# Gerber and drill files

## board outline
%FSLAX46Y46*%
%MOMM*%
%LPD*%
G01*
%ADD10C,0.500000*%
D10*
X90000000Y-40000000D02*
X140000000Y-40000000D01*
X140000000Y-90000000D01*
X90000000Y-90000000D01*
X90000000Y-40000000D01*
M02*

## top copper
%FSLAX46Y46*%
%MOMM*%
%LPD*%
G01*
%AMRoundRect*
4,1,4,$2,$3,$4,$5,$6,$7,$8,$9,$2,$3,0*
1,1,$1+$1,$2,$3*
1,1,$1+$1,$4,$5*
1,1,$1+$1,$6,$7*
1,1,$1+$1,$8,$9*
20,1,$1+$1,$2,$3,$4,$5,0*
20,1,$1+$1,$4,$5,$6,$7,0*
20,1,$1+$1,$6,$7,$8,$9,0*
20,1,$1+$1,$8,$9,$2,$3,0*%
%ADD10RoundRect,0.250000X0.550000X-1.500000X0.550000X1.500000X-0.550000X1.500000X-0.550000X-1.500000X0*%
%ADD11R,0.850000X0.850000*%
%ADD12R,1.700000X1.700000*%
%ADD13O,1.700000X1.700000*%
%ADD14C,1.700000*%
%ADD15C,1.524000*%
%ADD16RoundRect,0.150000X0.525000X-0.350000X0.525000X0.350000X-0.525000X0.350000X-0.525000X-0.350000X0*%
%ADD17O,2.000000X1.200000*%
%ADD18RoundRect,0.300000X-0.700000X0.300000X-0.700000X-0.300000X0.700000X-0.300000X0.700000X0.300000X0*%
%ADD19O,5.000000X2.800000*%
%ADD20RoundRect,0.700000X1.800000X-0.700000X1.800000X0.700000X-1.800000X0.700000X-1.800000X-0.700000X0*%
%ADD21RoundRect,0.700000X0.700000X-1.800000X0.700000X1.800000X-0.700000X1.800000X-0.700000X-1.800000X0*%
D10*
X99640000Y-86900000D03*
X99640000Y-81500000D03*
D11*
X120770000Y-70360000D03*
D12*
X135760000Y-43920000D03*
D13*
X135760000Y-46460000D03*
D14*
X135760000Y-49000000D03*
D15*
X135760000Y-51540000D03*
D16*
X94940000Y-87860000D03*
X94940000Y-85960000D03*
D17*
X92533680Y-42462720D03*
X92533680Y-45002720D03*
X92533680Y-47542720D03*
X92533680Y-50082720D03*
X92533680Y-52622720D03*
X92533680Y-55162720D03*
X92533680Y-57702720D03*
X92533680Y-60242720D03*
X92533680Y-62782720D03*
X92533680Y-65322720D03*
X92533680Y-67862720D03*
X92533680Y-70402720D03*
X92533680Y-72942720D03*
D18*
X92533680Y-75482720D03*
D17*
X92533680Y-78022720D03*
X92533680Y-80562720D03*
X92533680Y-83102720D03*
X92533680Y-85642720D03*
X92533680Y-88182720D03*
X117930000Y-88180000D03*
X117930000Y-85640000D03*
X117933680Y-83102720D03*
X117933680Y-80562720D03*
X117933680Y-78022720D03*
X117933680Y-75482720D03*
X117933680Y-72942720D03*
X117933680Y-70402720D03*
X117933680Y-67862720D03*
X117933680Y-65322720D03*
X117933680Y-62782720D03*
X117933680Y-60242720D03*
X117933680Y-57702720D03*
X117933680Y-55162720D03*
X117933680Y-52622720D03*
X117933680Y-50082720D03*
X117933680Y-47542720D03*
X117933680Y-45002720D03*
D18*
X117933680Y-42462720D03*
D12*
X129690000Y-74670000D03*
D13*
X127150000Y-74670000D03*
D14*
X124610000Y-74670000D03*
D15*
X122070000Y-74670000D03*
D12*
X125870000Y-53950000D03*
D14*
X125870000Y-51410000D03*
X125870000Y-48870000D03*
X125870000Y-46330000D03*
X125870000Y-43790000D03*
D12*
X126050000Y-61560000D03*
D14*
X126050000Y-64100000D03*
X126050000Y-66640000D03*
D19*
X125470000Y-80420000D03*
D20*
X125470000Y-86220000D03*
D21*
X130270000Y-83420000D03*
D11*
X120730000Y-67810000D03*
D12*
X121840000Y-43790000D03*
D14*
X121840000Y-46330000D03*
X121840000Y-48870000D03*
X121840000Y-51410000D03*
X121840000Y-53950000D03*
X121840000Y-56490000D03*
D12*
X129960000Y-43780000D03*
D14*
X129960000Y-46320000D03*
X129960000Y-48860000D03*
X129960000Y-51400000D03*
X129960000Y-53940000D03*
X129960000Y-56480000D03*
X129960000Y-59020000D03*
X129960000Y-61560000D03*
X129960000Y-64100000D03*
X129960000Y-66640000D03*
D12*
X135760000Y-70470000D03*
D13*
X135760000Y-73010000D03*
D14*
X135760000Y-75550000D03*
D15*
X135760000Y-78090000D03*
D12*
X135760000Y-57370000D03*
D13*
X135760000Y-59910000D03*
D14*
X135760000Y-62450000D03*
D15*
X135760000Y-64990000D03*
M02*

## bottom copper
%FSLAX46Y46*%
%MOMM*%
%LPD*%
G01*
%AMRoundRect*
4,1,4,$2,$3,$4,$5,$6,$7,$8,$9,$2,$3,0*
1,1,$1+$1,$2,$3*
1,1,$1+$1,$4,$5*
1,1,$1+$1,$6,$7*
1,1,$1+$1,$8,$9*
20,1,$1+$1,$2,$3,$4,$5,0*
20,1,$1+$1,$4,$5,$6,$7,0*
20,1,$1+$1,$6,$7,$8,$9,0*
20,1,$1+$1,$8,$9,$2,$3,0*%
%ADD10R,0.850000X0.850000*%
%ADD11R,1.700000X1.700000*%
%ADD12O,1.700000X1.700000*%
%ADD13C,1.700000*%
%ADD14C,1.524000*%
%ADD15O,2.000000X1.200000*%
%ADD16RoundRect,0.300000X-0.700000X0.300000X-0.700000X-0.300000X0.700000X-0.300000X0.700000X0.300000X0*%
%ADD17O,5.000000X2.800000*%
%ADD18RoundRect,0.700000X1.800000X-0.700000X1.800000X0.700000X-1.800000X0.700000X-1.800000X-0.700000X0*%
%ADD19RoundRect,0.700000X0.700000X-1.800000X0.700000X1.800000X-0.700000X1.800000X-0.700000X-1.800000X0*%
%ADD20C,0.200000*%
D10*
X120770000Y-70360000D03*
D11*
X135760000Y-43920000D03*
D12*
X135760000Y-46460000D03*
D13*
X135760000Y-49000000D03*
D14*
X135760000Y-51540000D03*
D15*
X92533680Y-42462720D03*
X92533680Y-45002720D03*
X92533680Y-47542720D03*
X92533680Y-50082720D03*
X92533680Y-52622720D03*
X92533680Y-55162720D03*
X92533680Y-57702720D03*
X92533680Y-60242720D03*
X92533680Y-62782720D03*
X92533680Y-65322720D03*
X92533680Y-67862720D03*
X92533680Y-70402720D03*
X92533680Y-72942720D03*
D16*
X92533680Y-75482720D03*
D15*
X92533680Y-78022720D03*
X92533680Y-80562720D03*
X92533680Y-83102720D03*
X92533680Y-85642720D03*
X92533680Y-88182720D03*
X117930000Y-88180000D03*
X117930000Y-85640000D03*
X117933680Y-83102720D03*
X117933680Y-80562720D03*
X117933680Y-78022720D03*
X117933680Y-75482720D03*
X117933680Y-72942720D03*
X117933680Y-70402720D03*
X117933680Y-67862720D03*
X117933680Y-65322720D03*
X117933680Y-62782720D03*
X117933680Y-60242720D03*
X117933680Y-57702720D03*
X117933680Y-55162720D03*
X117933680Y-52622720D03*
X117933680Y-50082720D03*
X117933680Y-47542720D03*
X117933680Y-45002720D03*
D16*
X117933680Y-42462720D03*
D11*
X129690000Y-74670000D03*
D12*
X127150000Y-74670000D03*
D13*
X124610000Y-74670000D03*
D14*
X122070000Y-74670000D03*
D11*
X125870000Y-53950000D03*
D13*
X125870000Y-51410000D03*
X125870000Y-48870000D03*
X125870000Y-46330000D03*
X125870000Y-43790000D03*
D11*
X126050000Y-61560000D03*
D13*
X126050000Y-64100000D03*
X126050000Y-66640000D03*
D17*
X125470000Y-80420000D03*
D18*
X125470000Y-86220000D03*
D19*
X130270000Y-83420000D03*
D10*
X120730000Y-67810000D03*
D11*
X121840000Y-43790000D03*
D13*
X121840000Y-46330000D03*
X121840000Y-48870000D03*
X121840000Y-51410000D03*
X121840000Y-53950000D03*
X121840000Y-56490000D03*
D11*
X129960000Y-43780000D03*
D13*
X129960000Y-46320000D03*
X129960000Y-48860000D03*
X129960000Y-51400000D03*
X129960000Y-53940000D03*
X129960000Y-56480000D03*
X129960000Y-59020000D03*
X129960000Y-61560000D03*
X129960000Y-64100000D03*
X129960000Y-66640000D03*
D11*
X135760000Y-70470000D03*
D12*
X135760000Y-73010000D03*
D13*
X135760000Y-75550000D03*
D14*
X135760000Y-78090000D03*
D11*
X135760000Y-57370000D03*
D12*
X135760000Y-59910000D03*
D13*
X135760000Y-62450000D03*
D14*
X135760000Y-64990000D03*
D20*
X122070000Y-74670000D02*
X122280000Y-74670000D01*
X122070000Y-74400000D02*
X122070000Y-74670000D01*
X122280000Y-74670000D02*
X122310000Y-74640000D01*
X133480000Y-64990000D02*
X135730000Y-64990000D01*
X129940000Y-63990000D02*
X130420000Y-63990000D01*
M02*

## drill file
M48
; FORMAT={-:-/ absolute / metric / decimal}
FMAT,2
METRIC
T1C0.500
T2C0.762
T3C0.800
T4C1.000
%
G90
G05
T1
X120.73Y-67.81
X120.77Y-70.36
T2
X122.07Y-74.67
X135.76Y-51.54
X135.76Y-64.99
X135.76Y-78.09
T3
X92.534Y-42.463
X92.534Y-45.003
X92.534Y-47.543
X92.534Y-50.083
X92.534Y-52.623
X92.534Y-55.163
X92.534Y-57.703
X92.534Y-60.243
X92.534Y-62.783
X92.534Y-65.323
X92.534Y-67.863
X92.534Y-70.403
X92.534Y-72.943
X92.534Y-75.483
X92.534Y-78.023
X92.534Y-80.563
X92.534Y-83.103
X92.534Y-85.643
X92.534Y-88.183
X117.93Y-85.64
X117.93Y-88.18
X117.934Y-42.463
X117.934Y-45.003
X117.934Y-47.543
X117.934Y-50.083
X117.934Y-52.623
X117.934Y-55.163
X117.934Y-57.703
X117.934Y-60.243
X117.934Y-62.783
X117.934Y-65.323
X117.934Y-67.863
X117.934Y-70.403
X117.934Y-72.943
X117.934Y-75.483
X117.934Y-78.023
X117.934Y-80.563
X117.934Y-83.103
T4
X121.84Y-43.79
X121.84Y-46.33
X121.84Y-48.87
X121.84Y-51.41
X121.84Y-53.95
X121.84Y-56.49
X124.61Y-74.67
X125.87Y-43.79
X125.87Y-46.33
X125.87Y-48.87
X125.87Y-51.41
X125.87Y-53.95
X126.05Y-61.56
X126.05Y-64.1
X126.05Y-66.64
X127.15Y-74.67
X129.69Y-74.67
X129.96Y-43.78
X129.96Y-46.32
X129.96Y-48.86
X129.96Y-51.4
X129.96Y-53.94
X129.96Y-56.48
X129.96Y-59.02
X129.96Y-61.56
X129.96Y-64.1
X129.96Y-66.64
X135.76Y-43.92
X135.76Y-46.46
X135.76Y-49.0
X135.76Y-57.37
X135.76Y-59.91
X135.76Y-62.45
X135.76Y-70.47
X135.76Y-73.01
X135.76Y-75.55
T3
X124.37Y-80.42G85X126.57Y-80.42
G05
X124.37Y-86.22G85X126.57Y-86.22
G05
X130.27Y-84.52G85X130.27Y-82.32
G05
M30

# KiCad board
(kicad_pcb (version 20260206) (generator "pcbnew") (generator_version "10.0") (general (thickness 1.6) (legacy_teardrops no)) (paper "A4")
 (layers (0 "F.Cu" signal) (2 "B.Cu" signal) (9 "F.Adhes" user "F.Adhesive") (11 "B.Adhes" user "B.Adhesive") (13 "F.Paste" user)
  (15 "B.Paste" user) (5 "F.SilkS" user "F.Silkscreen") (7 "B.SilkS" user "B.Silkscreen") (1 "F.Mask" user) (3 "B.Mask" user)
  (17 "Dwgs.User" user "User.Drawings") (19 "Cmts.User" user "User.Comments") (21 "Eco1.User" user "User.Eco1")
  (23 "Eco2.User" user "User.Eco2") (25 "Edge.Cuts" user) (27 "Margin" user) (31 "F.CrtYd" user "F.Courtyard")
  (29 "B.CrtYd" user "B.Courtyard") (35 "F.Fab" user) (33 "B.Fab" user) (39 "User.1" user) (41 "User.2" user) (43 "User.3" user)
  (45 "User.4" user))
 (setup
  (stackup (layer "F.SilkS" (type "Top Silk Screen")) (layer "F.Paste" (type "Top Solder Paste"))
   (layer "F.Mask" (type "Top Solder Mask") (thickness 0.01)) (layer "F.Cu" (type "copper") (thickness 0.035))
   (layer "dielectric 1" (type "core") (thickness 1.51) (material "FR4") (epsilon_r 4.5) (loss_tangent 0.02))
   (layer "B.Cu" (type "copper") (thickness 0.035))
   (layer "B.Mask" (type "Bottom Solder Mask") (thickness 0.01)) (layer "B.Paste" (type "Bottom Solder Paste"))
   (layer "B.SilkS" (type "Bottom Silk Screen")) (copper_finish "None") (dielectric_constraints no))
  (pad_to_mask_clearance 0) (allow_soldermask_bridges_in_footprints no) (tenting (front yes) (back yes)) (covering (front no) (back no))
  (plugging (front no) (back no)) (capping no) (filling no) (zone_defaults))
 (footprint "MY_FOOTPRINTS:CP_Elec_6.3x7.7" (layer "F.Cu") (at 99.64 84.2 90)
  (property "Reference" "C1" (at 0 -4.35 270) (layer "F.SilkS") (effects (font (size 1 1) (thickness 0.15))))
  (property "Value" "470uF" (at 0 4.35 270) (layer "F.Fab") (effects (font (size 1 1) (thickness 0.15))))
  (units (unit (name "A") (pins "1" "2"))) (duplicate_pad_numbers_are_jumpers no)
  (pad "1" smd roundrect (at -2.7 0 90) (size 3.5 1.6) (layers "F.Cu" "F.Mask" "F.Paste") (roundrect_rratio 0.15625) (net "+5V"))
  (pad "2" smd roundrect (at 2.7 0 90) (size 3.5 1.6) (layers "F.Cu" "F.Mask" "F.Paste") (roundrect_rratio 0.15625) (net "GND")))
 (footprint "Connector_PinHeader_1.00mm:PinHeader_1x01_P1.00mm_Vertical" (layer "F.Cu") (at 120.77 70.36)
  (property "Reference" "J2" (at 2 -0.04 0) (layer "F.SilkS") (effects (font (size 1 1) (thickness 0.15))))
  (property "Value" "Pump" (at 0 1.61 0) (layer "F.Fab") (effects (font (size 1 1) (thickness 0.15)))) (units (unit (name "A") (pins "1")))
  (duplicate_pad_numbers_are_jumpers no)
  (pad "1" thru_hole rect (at 0 0) (size 0.85 0.85) (drill 0.5) (layers "*.Cu" "*.Mask") (remove_unused_layers no) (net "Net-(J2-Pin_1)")))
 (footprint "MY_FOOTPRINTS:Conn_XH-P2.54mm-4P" (layer "F.Cu") (at 135.76 47.73)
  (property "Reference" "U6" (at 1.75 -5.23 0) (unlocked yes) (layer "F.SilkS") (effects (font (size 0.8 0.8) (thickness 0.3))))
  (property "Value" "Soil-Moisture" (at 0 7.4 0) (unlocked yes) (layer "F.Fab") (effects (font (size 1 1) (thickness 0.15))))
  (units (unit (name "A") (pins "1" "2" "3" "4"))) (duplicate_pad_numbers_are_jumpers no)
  (pad "1" thru_hole rect (at 0 -3.81) (size 1.7 1.7) (drill 1) (layers "*.Cu" "*.Mask") (remove_unused_layers no) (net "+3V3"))
  (pad "2" thru_hole oval (at 0 -1.27) (size 1.7 1.7) (drill 1) (layers "*.Cu" "*.Mask") (remove_unused_layers no) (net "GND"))
  (pad "3" thru_hole circle (at 0 1.27) (size 1.7 1.7) (drill 1) (layers "*.Cu" "*.Mask") (remove_unused_layers no)
   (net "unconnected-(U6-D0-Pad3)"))
  (pad "4" thru_hole circle (at 0 3.81) (size 1.524 1.524) (drill 0.762) (layers "*.Cu" "*.Mask") (remove_unused_layers no)
   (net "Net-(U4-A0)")))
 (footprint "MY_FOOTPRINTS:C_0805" (layer "F.Cu") (at 94.94 86.91 90)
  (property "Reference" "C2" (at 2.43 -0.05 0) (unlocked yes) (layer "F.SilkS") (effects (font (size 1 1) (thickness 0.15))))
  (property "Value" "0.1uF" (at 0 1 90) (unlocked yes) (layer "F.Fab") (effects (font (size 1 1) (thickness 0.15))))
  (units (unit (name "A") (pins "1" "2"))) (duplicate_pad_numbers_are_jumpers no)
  (pad "1" smd roundrect (at -0.95 0 90) (size 1 1.35) (layers "F.Cu" "F.Mask" "F.Paste") (roundrect_rratio 0.15) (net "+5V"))
  (pad "2" smd roundrect (at 0.95 0 90) (size 1 1.35) (layers "F.Cu" "F.Mask" "F.Paste") (roundrect_rratio 0.15) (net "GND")))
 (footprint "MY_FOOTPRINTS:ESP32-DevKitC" (layer "F.Cu") (at 92.53 42.46)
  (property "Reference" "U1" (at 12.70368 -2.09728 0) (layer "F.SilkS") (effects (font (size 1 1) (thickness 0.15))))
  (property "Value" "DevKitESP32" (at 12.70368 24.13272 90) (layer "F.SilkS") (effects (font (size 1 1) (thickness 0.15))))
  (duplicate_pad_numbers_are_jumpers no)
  (pad "1" thru_hole oval (at 0.00368 0.00272 270) (size 1.2 2) (drill 0.8) (layers "*.Cu" "*.Mask") (remove_unused_layers no) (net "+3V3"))
  (pad "2" thru_hole oval (at 0.00368 2.54272 270) (size 1.2 2) (drill 0.8) (layers "*.Cu" "*.Mask") (remove_unused_layers no)
   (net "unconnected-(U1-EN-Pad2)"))
  (pad "3" thru_hole oval (at 0.00368 5.08272 270) (size 1.2 2) (drill 0.8) (layers "*.Cu" "*.Mask") (remove_unused_layers no)
   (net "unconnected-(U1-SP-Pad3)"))
  (pad "4" thru_hole oval (at 0.00368 7.62272 270) (size 1.2 2) (drill 0.8) (layers "*.Cu" "*.Mask") (remove_unused_layers no)
   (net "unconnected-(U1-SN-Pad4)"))
  (pad "5" thru_hole oval (at 0.00368 10.16272 270) (size 1.2 2) (drill 0.8) (layers "*.Cu" "*.Mask") (remove_unused_layers no)
   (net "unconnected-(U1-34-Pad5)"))
  (pad "6" thru_hole oval (at 0.00368 12.70272 270) (size 1.2 2) (drill 0.8) (layers "*.Cu" "*.Mask") (remove_unused_layers no)
   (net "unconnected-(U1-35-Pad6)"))
  (pad "7" thru_hole oval (at 0.00368 15.24272 270) (size 1.2 2) (drill 0.8) (layers "*.Cu" "*.Mask") (remove_unused_layers no)
   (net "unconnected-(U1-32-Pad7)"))
  (pad "8" thru_hole oval (at 0.00368 17.78272 270) (size 1.2 2) (drill 0.8) (layers "*.Cu" "*.Mask") (remove_unused_layers no)
   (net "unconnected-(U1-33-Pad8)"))
  (pad "9" thru_hole oval (at 0.00368 20.32272 270) (size 1.2 2) (drill 0.8) (layers "*.Cu" "*.Mask") (remove_unused_layers no)
   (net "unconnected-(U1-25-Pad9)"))
  (pad "10" thru_hole oval (at 0.00368 22.86272 270) (size 1.2 2) (drill 0.8) (layers "*.Cu" "*.Mask") (remove_unused_layers no)
   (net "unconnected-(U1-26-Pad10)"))
  (pad "11" thru_hole oval (at 0.00368 25.40272 270) (size 1.2 2) (drill 0.8) (layers "*.Cu" "*.Mask") (remove_unused_layers no)
   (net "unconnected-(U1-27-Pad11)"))
  (pad "12" thru_hole oval (at 0.00368 27.94272 270) (size 1.2 2) (drill 0.8) (layers "*.Cu" "*.Mask") (remove_unused_layers no)
   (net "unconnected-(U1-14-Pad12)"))
  (pad "13" thru_hole oval (at 0.00368 30.48272 270) (size 1.2 2) (drill 0.8) (layers "*.Cu" "*.Mask") (remove_unused_layers no)
   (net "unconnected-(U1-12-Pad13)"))
  (pad "14" thru_hole roundrect (at 0.00368 33.02272 270) (size 1.2 2) (drill 0.8) (layers "*.Cu" "*.Mask") (remove_unused_layers no)
   (roundrect_rratio 0.25) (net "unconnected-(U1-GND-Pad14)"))
  (pad "15" thru_hole oval (at 0.00368 35.56272 270) (size 1.2 2) (drill 0.8) (layers "*.Cu" "*.Mask") (remove_unused_layers no)
   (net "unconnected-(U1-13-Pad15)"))
  (pad "16" thru_hole oval (at 0.00368 38.10272 270) (size 1.2 2) (drill 0.8) (layers "*.Cu" "*.Mask") (remove_unused_layers no)
   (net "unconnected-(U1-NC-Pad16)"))
  (pad "17" thru_hole oval (at 0.00368 40.64272 270) (size 1.2 2) (drill 0.8) (layers "*.Cu" "*.Mask") (remove_unused_layers no)
   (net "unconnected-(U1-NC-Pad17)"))
  (pad "18" thru_hole oval (at 0.00368 43.18272 270) (size 1.2 2) (drill 0.8) (layers "*.Cu" "*.Mask") (remove_unused_layers no) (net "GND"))
  (pad "19" thru_hole oval (at 0.00368 45.72272 270) (size 1.2 2) (drill 0.8) (layers "*.Cu" "*.Mask") (remove_unused_layers no) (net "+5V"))
  (pad "20" thru_hole oval (at 25.4 45.72 270) (size 1.2 2) (drill 0.8) (layers "*.Cu" "*.Mask") (remove_unused_layers no)
   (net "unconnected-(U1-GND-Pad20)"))
  (pad "21" thru_hole oval (at 25.4 43.18 270) (size 1.2 2) (drill 0.8) (layers "*.Cu" "*.Mask") (remove_unused_layers no)
   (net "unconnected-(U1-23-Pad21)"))
  (pad "22" thru_hole oval (at 25.40368 40.64272 270) (size 1.2 2) (drill 0.8) (layers "*.Cu" "*.Mask") (remove_unused_layers no)
   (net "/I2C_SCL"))
  (pad "23" thru_hole oval (at 25.40368 38.10272 270) (size 1.2 2) (drill 0.8) (layers "*.Cu" "*.Mask") (remove_unused_layers no)
   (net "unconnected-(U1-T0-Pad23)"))
  (pad "24" thru_hole oval (at 25.40368 35.56272 270) (size 1.2 2) (drill 0.8) (layers "*.Cu" "*.Mask") (remove_unused_layers no)
   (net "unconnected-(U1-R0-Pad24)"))
  (pad "25" thru_hole oval (at 25.40368 33.02272 270) (size 1.2 2) (drill 0.8) (layers "*.Cu" "*.Mask") (remove_unused_layers no)
   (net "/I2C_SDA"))
  (pad "26" thru_hole oval (at 25.40368 30.48272 270) (size 1.2 2) (drill 0.8) (layers "*.Cu" "*.Mask") (remove_unused_layers no)
   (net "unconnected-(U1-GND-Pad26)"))
  (pad "27" thru_hole oval (at 25.40368 27.94272 270) (size 1.2 2) (drill 0.8) (layers "*.Cu" "*.Mask") (remove_unused_layers no)
   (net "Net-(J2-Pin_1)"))
  (pad "28" thru_hole oval (at 25.40368 25.40272 270) (size 1.2 2) (drill 0.8) (layers "*.Cu" "*.Mask") (remove_unused_layers no)
   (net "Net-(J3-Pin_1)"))
  (pad "29" thru_hole oval (at 25.40368 22.86272 270) (size 1.2 2) (drill 0.8) (layers "*.Cu" "*.Mask") (remove_unused_layers no)
   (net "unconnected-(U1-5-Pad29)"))
  (pad "30" thru_hole oval (at 25.40368 20.32272 270) (size 1.2 2) (drill 0.8) (layers "*.Cu" "*.Mask") (remove_unused_layers no)
   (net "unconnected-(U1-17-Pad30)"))
  (pad "31" thru_hole oval (at 25.40368 17.78272 270) (size 1.2 2) (drill 0.8) (layers "*.Cu" "*.Mask") (remove_unused_layers no)
   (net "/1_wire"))
  (pad "32" thru_hole oval (at 25.40368 15.24272 270) (size 1.2 2) (drill 0.8) (layers "*.Cu" "*.Mask") (remove_unused_layers no)
   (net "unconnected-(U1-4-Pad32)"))
  (pad "33" thru_hole oval (at 25.40368 12.70272 270) (size 1.2 2) (drill 0.8) (layers "*.Cu" "*.Mask") (remove_unused_layers no)
   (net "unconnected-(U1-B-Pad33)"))
  (pad "34" thru_hole oval (at 25.40368 10.16272 270) (size 1.2 2) (drill 0.8) (layers "*.Cu" "*.Mask") (remove_unused_layers no)
   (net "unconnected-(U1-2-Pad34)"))
  (pad "35" thru_hole oval (at 25.40368 7.62272 270) (size 1.2 2) (drill 0.8) (layers "*.Cu" "*.Mask") (remove_unused_layers no)
   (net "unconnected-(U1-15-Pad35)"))
  (pad "36" thru_hole oval (at 25.40368 5.08272 270) (size 1.2 2) (drill 0.8) (layers "*.Cu" "*.Mask") (remove_unused_layers no)
   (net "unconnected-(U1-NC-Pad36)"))
  (pad "37" thru_hole oval (at 25.40368 2.54272 270) (size 1.2 2) (drill 0.8) (layers "*.Cu" "*.Mask") (remove_unused_layers no)
   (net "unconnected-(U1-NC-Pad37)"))
  (pad "38" thru_hole roundrect (at 25.40368 0.00272 270) (size 1.2 2) (drill 0.8) (layers "*.Cu" "*.Mask") (remove_unused_layers no)
   (roundrect_rratio 0.25) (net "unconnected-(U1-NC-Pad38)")))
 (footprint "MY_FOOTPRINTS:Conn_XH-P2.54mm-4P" (layer "F.Cu") (at 125.88 74.67 -90)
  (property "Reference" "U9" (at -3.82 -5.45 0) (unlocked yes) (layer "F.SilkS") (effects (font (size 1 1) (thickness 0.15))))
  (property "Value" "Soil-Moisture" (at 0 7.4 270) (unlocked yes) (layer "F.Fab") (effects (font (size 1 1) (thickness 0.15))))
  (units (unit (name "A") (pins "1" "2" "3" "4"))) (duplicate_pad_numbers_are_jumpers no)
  (pad "1" thru_hole rect (at 0 -3.81 270) (size 1.7 1.7) (drill 1) (layers "*.Cu" "*.Mask") (remove_unused_layers no) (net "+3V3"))
  (pad "2" thru_hole oval (at 0 -1.27 270) (size 1.7 1.7) (drill 1) (layers "*.Cu" "*.Mask") (remove_unused_layers no) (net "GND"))
  (pad "3" thru_hole circle (at 0 1.27 270) (size 1.7 1.7) (drill 1) (layers "*.Cu" "*.Mask") (remove_unused_layers no)
   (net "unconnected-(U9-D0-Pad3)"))
  (pad "4" thru_hole circle (at 0 3.81 270) (size 1.524 1.524) (drill 0.762) (layers "*.Cu" "*.Mask") (remove_unused_layers no)
   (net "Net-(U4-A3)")))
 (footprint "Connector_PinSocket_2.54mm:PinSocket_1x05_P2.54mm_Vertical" (layer "F.Cu") (at 125.87 53.95 180)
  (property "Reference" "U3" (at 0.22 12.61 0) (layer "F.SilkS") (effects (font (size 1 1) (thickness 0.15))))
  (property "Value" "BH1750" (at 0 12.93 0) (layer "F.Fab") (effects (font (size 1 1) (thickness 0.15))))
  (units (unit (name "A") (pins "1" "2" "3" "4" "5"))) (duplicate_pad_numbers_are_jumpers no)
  (pad "1" thru_hole rect (at 0 0 180) (size 1.7 1.7) (drill 1) (layers "*.Cu" "*.Mask") (remove_unused_layers no) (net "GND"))
  (pad "2" thru_hole circle (at 0 2.54 180) (size 1.7 1.7) (drill 1) (layers "*.Cu" "*.Mask") (remove_unused_layers no)
   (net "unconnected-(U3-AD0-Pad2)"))
  (pad "3" thru_hole circle (at 0 5.08 180) (size 1.7 1.7) (drill 1) (layers "*.Cu" "*.Mask") (remove_unused_layers no) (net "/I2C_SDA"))
  (pad "4" thru_hole circle (at 0 7.62 180) (size 1.7 1.7) (drill 1) (layers "*.Cu" "*.Mask") (remove_unused_layers no) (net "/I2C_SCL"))
  (pad "5" thru_hole circle (at 0 10.16 180) (size 1.7 1.7) (drill 1) (layers "*.Cu" "*.Mask") (remove_unused_layers no) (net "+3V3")))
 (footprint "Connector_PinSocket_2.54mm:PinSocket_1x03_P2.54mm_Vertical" (layer "F.Cu") (at 126.05 61.56)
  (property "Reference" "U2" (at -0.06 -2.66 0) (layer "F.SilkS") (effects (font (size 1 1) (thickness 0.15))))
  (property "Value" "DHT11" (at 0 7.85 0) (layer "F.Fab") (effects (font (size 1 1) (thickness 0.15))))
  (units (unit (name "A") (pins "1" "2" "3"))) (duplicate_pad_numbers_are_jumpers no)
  (pad "1" thru_hole rect (at 0 0) (size 1.7 1.7) (drill 1) (layers "*.Cu" "*.Mask") (remove_unused_layers no) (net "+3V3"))
  (pad "2" thru_hole circle (at 0 2.54) (size 1.7 1.7) (drill 1) (layers "*.Cu" "*.Mask") (remove_unused_layers no) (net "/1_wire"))
  (pad "3" thru_hole circle (at 0 5.08) (size 1.7 1.7) (drill 1) (layers "*.Cu" "*.Mask") (remove_unused_layers no) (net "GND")))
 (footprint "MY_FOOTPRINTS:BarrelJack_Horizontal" (layer "F.Cu") (at 125.47 80.42 90)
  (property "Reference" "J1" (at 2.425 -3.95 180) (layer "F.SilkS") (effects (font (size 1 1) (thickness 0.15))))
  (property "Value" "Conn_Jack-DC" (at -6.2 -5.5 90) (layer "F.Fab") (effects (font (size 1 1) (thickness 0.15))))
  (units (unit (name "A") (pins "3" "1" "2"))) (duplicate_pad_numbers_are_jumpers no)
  (pad "1" thru_hole oval (at 0 0 90) (size 2.8 5) (drill oval 0.8 3) (layers "*.Cu" "*.Mask") (remove_unused_layers no) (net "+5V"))
  (pad "2" thru_hole roundrect (at -5.8 0 90) (size 2.8 5) (drill oval 0.8 3) (layers "*.Cu" "*.Mask") (remove_unused_layers no)
   (roundrect_rratio 0.25) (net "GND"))
  (pad "3" thru_hole roundrect (at -3 4.8 90) (size 5 2.8) (drill oval 3 0.8) (layers "*.Cu" "*.Mask") (remove_unused_layers no)
   (roundrect_rratio 0.25) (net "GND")))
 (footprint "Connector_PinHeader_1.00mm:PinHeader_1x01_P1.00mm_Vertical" (layer "F.Cu") (at 120.73 67.81)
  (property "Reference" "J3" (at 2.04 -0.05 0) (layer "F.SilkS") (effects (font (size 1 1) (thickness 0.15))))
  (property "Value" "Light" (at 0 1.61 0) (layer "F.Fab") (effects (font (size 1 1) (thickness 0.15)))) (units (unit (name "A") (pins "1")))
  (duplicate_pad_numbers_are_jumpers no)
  (pad "1" thru_hole rect (at 0 0) (size 0.85 0.85) (drill 0.5) (layers "*.Cu" "*.Mask") (remove_unused_layers no) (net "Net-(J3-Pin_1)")))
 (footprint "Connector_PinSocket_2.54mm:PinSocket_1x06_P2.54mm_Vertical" (layer "F.Cu") (at 121.84 43.79)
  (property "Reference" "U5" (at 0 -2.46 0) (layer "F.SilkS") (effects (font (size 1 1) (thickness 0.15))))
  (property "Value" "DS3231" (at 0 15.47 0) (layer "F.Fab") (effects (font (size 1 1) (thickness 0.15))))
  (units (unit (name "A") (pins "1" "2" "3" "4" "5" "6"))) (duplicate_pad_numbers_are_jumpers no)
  (pad "1" thru_hole rect (at 0 0) (size 1.7 1.7) (drill 1) (layers "*.Cu" "*.Mask") (remove_unused_layers no)
   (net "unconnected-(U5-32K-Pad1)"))
  (pad "2" thru_hole circle (at 0 2.54) (size 1.7 1.7) (drill 1) (layers "*.Cu" "*.Mask") (remove_unused_layers no)
   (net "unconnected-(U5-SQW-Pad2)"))
  (pad "3" thru_hole circle (at 0 5.08) (size 1.7 1.7) (drill 1) (layers "*.Cu" "*.Mask") (remove_unused_layers no) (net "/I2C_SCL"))
  (pad "4" thru_hole circle (at 0 7.62) (size 1.7 1.7) (drill 1) (layers "*.Cu" "*.Mask") (remove_unused_layers no) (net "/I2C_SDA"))
  (pad "5" thru_hole circle (at 0 10.16) (size 1.7 1.7) (drill 1) (layers "*.Cu" "*.Mask") (remove_unused_layers no) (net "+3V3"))
  (pad "6" thru_hole circle (at 0 12.7) (size 1.7 1.7) (drill 1) (layers "*.Cu" "*.Mask") (remove_unused_layers no) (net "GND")))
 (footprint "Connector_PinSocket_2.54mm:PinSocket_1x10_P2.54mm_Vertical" (layer "F.Cu") (at 129.96 43.78)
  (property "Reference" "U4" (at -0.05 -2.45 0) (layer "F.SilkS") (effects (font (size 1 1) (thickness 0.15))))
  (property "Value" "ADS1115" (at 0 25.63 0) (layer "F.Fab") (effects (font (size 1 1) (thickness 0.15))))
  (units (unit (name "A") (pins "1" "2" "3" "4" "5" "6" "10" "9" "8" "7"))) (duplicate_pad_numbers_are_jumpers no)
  (pad "1" thru_hole rect (at 0 0) (size 1.7 1.7) (drill 1) (layers "*.Cu" "*.Mask") (remove_unused_layers no) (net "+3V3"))
  (pad "2" thru_hole circle (at 0 2.54) (size 1.7 1.7) (drill 1) (layers "*.Cu" "*.Mask") (remove_unused_layers no) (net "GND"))
  (pad "3" thru_hole circle (at 0 5.08) (size 1.7 1.7) (drill 1) (layers "*.Cu" "*.Mask") (remove_unused_layers no) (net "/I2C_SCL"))
  (pad "4" thru_hole circle (at 0 7.62) (size 1.7 1.7) (drill 1) (layers "*.Cu" "*.Mask") (remove_unused_layers no) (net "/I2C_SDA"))
  (pad "5" thru_hole circle (at 0 10.16) (size 1.7 1.7) (drill 1) (layers "*.Cu" "*.Mask") (remove_unused_layers no)
   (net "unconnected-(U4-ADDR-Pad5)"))
  (pad "6" thru_hole circle (at 0 12.7) (size 1.7 1.7) (drill 1) (layers "*.Cu" "*.Mask") (remove_unused_layers no)
   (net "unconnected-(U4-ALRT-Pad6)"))
  (pad "7" thru_hole circle (at 0 15.24) (size 1.7 1.7) (drill 1) (layers "*.Cu" "*.Mask") (remove_unused_layers no) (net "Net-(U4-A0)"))
  (pad "8" thru_hole circle (at 0 17.78) (size 1.7 1.7) (drill 1) (layers "*.Cu" "*.Mask") (remove_unused_layers no) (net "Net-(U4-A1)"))
  (pad "9" thru_hole circle (at 0 20.32) (size 1.7 1.7) (drill 1) (layers "*.Cu" "*.Mask") (remove_unused_layers no) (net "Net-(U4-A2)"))
  (pad "10" thru_hole circle (at 0 22.86) (size 1.7 1.7) (drill 1) (layers "*.Cu" "*.Mask") (remove_unused_layers no) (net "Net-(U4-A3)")))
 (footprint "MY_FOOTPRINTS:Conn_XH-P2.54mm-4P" (layer "F.Cu") (at 135.76 74.28)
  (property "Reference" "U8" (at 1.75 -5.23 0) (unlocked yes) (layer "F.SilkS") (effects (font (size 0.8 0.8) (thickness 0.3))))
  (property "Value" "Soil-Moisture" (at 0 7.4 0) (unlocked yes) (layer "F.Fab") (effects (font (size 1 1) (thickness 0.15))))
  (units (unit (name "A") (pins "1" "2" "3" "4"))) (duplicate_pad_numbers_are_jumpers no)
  (pad "1" thru_hole rect (at 0 -3.81) (size 1.7 1.7) (drill 1) (layers "*.Cu" "*.Mask") (remove_unused_layers no) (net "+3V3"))
  (pad "2" thru_hole oval (at 0 -1.27) (size 1.7 1.7) (drill 1) (layers "*.Cu" "*.Mask") (remove_unused_layers no) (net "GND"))
  (pad "3" thru_hole circle (at 0 1.27) (size 1.7 1.7) (drill 1) (layers "*.Cu" "*.Mask") (remove_unused_layers no)
   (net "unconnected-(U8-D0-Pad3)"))
  (pad "4" thru_hole circle (at 0 3.81) (size 1.524 1.524) (drill 0.762) (layers "*.Cu" "*.Mask") (remove_unused_layers no)
   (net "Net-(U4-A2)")))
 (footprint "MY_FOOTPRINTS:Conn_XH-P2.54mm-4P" (layer "F.Cu") (at 135.76 61.18)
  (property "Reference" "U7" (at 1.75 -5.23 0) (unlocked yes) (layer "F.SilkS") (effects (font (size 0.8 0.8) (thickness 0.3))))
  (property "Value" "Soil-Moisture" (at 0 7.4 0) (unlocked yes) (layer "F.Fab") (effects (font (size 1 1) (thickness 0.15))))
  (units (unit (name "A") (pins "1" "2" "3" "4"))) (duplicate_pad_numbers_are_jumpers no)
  (pad "1" thru_hole rect (at 0 -3.81) (size 1.7 1.7) (drill 1) (layers "*.Cu" "*.Mask") (remove_unused_layers no) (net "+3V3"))
  (pad "2" thru_hole oval (at 0 -1.27) (size 1.7 1.7) (drill 1) (layers "*.Cu" "*.Mask") (remove_unused_layers no) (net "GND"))
  (pad "3" thru_hole circle (at 0 1.27) (size 1.7 1.7) (drill 1) (layers "*.Cu" "*.Mask") (remove_unused_layers no)
   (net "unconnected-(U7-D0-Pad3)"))
  (pad "4" thru_hole circle (at 0 3.81) (size 1.524 1.524) (drill 0.762) (layers "*.Cu" "*.Mask") (remove_unused_layers no)
   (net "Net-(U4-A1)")))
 (gr_rect (start 90 40) (end 140 90) (stroke (width 0.5) (type solid)) (fill no) (layer "Edge.Cuts"))
 (segment (start 122.07 74.67) (end 122.28 74.67) (width 0.2) (layer "B.Cu") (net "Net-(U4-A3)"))
 (segment (start 122.07 74.4) (end 122.07 74.67) (width 0.2) (layer "B.Cu") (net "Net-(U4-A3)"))
 (segment (start 122.28 74.67) (end 122.31 74.64) (width 0.2) (layer "B.Cu") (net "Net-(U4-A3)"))
 (segment (start 133.48 64.99) (end 135.73 64.99) (width 0.2) (layer "B.Cu") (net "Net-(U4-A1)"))
 (segment (start 129.94 63.99) (end 130.42 63.99) (width 0.2) (layer "B.Cu") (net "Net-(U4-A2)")))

